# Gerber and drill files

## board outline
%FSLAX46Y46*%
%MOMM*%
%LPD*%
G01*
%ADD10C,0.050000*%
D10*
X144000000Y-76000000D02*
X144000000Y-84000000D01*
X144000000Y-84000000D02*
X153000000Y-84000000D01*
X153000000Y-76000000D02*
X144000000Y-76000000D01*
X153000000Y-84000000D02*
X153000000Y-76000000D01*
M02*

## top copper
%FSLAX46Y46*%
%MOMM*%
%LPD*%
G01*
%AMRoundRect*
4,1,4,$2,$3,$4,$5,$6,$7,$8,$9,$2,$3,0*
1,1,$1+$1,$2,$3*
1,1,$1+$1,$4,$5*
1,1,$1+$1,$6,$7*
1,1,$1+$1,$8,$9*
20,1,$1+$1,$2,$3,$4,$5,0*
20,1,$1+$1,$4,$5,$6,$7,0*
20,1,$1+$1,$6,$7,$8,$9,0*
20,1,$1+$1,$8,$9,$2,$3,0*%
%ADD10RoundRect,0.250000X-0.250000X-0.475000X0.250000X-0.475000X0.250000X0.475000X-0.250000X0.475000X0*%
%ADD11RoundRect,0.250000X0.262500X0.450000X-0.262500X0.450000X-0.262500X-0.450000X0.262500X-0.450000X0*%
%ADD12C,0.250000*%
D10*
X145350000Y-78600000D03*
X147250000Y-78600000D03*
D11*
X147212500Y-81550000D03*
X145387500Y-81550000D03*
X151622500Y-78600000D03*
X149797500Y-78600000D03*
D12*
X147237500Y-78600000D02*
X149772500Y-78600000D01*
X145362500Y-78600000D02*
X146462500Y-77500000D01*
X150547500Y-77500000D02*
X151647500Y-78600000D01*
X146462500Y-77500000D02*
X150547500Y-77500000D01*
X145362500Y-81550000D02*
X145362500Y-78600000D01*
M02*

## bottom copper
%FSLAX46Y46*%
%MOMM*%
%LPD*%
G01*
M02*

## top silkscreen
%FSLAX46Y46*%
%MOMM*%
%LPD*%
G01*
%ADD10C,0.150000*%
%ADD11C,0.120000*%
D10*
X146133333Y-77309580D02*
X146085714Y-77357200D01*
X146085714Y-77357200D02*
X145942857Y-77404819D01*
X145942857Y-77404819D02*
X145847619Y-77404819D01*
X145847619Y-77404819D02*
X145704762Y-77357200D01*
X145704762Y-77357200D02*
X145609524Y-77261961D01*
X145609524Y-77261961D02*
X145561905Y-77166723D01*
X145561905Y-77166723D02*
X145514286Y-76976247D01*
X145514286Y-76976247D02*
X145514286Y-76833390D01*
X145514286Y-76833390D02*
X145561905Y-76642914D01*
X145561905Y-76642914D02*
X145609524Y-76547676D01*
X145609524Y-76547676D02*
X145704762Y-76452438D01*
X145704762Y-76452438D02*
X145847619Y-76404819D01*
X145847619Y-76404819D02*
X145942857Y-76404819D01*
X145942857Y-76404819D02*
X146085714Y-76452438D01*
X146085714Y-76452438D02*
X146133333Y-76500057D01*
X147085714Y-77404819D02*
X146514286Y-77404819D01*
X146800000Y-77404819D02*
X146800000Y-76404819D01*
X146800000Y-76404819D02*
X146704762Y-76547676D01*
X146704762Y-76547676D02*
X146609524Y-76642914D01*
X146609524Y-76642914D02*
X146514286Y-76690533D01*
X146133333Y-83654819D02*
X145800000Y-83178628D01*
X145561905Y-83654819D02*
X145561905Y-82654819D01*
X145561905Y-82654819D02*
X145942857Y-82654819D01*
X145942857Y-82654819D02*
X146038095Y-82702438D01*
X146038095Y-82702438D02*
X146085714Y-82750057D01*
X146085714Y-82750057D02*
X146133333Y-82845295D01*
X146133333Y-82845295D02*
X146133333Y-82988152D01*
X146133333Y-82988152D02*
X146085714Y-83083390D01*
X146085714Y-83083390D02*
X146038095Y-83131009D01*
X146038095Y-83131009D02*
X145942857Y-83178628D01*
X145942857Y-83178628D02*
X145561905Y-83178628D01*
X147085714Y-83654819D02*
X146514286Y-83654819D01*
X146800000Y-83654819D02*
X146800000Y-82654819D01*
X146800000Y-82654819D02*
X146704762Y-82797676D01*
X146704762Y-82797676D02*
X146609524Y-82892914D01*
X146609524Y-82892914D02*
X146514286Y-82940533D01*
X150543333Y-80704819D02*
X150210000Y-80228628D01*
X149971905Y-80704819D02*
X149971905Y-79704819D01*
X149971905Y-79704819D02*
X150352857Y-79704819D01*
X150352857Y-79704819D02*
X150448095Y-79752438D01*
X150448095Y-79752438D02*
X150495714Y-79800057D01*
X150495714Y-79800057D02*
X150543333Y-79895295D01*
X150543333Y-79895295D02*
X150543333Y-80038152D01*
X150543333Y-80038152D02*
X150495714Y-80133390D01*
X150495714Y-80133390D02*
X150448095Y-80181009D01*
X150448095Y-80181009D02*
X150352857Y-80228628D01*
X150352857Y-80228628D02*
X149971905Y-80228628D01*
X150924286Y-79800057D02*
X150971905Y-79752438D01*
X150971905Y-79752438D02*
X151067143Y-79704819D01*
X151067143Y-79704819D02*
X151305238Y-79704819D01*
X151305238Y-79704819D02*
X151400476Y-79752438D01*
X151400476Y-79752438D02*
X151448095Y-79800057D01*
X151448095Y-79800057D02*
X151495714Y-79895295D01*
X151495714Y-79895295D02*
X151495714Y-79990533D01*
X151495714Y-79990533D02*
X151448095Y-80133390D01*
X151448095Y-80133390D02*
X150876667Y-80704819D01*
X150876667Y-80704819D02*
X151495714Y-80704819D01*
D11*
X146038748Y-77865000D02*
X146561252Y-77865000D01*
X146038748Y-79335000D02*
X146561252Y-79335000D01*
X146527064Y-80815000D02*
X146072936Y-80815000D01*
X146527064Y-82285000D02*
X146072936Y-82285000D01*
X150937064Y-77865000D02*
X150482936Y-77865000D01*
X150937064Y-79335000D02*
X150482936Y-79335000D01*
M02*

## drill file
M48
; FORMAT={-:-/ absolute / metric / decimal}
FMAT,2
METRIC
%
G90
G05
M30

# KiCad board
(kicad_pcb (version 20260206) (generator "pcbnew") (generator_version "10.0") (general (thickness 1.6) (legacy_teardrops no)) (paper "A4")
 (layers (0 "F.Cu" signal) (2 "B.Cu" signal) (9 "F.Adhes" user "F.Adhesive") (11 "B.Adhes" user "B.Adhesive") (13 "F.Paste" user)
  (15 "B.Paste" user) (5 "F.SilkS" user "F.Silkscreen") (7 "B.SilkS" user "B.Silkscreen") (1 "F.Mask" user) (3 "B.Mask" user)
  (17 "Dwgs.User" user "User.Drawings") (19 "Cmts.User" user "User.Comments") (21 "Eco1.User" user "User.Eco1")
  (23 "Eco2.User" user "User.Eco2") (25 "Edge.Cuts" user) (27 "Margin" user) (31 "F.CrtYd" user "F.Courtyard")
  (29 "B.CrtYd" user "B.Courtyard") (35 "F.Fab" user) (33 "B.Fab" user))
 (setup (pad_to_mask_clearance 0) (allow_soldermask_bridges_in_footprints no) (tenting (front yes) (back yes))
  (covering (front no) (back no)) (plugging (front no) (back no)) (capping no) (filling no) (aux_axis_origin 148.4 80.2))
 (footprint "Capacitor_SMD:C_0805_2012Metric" (layer "F.Cu") (at 146.3 78.6)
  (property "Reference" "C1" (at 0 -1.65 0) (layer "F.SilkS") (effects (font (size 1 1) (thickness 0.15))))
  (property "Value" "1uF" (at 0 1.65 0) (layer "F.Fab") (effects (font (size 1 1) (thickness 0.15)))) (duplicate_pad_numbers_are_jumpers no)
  (fp_line (start -0.261252 -0.735) (end 0.261252 -0.735) (stroke (width 0.12) (type solid)) (layer "F.SilkS"))
  (fp_line (start -0.261252 0.735) (end 0.261252 0.735) (stroke (width 0.12) (type solid)) (layer "F.SilkS"))
  (pad "1" smd roundrect (at -0.95 0) (size 1 1.45) (layers "F.Cu" "F.Mask" "F.Paste") (roundrect_rratio 0.25) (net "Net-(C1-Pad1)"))
  (pad "2" smd roundrect (at 0.95 0) (size 1 1.45) (layers "F.Cu" "F.Mask" "F.Paste") (roundrect_rratio 0.25) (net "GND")))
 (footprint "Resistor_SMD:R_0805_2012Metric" (layer "F.Cu") (at 146.3 81.55 180)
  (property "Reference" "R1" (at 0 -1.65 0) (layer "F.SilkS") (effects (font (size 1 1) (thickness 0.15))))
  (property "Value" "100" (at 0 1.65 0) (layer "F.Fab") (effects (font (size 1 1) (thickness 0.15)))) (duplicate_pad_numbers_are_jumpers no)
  (fp_line (start -0.227064 0.735) (end 0.227064 0.735) (stroke (width 0.12) (type solid)) (layer "F.SilkS"))
  (fp_line (start -0.227064 -0.735) (end 0.227064 -0.735) (stroke (width 0.12) (type solid)) (layer "F.SilkS"))
  (pad "1" smd roundrect (at -0.9125 0 180) (size 1.025 1.4) (layers "F.Cu" "F.Mask" "F.Paste") (roundrect_rratio 0.243902) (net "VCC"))
  (pad "2" smd roundrect (at 0.9125 0 180) (size 1.025 1.4) (layers "F.Cu" "F.Mask" "F.Paste") (roundrect_rratio 0.243902)
   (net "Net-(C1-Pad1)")))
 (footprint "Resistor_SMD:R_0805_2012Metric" (layer "F.Cu") (at 150.71 78.6 180)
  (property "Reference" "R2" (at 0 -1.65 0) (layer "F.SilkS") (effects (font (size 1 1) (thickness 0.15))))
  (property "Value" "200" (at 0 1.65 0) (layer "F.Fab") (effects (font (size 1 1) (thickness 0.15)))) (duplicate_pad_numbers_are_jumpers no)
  (fp_line (start -0.227064 0.735) (end 0.227064 0.735) (stroke (width 0.12) (type solid)) (layer "F.SilkS"))
  (fp_line (start -0.227064 -0.735) (end 0.227064 -0.735) (stroke (width 0.12) (type solid)) (layer "F.SilkS"))
  (pad "1" smd roundrect (at -0.9125 0 180) (size 1.025 1.4) (layers "F.Cu" "F.Mask" "F.Paste") (roundrect_rratio 0.243902)
   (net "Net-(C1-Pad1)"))
  (pad "2" smd roundrect (at 0.9125 0 180) (size 1.025 1.4) (layers "F.Cu" "F.Mask" "F.Paste") (roundrect_rratio 0.243902) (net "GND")))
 (gr_line (start 144 76) (end 144 84) (stroke (width 0.05) (type solid)) (layer "Edge.Cuts"))
 (gr_line (start 144 84) (end 153 84) (stroke (width 0.05) (type solid)) (layer "Edge.Cuts"))
 (gr_line (start 153 76) (end 144 76) (stroke (width 0.05) (type solid)) (layer "Edge.Cuts"))
 (gr_line (start 153 84) (end 153 76) (stroke (width 0.05) (type solid)) (layer "Edge.Cuts"))
 (segment (start 147.2375 78.6) (end 149.7725 78.6) (width 0.25) (layer "F.Cu") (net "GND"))
 (segment (start 145.3625 78.6) (end 146.4625 77.5) (width 0.25) (layer "F.Cu") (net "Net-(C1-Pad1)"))
 (segment (start 150.5475 77.5) (end 151.6475 78.6) (width 0.25) (layer "F.Cu") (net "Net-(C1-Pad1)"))
 (segment (start 146.4625 77.5) (end 150.5475 77.5) (width 0.25) (layer "F.Cu") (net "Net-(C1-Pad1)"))
 (segment (start 145.3625 81.55) (end 145.3625 78.6) (width 0.25) (layer "F.Cu") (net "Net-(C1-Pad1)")))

